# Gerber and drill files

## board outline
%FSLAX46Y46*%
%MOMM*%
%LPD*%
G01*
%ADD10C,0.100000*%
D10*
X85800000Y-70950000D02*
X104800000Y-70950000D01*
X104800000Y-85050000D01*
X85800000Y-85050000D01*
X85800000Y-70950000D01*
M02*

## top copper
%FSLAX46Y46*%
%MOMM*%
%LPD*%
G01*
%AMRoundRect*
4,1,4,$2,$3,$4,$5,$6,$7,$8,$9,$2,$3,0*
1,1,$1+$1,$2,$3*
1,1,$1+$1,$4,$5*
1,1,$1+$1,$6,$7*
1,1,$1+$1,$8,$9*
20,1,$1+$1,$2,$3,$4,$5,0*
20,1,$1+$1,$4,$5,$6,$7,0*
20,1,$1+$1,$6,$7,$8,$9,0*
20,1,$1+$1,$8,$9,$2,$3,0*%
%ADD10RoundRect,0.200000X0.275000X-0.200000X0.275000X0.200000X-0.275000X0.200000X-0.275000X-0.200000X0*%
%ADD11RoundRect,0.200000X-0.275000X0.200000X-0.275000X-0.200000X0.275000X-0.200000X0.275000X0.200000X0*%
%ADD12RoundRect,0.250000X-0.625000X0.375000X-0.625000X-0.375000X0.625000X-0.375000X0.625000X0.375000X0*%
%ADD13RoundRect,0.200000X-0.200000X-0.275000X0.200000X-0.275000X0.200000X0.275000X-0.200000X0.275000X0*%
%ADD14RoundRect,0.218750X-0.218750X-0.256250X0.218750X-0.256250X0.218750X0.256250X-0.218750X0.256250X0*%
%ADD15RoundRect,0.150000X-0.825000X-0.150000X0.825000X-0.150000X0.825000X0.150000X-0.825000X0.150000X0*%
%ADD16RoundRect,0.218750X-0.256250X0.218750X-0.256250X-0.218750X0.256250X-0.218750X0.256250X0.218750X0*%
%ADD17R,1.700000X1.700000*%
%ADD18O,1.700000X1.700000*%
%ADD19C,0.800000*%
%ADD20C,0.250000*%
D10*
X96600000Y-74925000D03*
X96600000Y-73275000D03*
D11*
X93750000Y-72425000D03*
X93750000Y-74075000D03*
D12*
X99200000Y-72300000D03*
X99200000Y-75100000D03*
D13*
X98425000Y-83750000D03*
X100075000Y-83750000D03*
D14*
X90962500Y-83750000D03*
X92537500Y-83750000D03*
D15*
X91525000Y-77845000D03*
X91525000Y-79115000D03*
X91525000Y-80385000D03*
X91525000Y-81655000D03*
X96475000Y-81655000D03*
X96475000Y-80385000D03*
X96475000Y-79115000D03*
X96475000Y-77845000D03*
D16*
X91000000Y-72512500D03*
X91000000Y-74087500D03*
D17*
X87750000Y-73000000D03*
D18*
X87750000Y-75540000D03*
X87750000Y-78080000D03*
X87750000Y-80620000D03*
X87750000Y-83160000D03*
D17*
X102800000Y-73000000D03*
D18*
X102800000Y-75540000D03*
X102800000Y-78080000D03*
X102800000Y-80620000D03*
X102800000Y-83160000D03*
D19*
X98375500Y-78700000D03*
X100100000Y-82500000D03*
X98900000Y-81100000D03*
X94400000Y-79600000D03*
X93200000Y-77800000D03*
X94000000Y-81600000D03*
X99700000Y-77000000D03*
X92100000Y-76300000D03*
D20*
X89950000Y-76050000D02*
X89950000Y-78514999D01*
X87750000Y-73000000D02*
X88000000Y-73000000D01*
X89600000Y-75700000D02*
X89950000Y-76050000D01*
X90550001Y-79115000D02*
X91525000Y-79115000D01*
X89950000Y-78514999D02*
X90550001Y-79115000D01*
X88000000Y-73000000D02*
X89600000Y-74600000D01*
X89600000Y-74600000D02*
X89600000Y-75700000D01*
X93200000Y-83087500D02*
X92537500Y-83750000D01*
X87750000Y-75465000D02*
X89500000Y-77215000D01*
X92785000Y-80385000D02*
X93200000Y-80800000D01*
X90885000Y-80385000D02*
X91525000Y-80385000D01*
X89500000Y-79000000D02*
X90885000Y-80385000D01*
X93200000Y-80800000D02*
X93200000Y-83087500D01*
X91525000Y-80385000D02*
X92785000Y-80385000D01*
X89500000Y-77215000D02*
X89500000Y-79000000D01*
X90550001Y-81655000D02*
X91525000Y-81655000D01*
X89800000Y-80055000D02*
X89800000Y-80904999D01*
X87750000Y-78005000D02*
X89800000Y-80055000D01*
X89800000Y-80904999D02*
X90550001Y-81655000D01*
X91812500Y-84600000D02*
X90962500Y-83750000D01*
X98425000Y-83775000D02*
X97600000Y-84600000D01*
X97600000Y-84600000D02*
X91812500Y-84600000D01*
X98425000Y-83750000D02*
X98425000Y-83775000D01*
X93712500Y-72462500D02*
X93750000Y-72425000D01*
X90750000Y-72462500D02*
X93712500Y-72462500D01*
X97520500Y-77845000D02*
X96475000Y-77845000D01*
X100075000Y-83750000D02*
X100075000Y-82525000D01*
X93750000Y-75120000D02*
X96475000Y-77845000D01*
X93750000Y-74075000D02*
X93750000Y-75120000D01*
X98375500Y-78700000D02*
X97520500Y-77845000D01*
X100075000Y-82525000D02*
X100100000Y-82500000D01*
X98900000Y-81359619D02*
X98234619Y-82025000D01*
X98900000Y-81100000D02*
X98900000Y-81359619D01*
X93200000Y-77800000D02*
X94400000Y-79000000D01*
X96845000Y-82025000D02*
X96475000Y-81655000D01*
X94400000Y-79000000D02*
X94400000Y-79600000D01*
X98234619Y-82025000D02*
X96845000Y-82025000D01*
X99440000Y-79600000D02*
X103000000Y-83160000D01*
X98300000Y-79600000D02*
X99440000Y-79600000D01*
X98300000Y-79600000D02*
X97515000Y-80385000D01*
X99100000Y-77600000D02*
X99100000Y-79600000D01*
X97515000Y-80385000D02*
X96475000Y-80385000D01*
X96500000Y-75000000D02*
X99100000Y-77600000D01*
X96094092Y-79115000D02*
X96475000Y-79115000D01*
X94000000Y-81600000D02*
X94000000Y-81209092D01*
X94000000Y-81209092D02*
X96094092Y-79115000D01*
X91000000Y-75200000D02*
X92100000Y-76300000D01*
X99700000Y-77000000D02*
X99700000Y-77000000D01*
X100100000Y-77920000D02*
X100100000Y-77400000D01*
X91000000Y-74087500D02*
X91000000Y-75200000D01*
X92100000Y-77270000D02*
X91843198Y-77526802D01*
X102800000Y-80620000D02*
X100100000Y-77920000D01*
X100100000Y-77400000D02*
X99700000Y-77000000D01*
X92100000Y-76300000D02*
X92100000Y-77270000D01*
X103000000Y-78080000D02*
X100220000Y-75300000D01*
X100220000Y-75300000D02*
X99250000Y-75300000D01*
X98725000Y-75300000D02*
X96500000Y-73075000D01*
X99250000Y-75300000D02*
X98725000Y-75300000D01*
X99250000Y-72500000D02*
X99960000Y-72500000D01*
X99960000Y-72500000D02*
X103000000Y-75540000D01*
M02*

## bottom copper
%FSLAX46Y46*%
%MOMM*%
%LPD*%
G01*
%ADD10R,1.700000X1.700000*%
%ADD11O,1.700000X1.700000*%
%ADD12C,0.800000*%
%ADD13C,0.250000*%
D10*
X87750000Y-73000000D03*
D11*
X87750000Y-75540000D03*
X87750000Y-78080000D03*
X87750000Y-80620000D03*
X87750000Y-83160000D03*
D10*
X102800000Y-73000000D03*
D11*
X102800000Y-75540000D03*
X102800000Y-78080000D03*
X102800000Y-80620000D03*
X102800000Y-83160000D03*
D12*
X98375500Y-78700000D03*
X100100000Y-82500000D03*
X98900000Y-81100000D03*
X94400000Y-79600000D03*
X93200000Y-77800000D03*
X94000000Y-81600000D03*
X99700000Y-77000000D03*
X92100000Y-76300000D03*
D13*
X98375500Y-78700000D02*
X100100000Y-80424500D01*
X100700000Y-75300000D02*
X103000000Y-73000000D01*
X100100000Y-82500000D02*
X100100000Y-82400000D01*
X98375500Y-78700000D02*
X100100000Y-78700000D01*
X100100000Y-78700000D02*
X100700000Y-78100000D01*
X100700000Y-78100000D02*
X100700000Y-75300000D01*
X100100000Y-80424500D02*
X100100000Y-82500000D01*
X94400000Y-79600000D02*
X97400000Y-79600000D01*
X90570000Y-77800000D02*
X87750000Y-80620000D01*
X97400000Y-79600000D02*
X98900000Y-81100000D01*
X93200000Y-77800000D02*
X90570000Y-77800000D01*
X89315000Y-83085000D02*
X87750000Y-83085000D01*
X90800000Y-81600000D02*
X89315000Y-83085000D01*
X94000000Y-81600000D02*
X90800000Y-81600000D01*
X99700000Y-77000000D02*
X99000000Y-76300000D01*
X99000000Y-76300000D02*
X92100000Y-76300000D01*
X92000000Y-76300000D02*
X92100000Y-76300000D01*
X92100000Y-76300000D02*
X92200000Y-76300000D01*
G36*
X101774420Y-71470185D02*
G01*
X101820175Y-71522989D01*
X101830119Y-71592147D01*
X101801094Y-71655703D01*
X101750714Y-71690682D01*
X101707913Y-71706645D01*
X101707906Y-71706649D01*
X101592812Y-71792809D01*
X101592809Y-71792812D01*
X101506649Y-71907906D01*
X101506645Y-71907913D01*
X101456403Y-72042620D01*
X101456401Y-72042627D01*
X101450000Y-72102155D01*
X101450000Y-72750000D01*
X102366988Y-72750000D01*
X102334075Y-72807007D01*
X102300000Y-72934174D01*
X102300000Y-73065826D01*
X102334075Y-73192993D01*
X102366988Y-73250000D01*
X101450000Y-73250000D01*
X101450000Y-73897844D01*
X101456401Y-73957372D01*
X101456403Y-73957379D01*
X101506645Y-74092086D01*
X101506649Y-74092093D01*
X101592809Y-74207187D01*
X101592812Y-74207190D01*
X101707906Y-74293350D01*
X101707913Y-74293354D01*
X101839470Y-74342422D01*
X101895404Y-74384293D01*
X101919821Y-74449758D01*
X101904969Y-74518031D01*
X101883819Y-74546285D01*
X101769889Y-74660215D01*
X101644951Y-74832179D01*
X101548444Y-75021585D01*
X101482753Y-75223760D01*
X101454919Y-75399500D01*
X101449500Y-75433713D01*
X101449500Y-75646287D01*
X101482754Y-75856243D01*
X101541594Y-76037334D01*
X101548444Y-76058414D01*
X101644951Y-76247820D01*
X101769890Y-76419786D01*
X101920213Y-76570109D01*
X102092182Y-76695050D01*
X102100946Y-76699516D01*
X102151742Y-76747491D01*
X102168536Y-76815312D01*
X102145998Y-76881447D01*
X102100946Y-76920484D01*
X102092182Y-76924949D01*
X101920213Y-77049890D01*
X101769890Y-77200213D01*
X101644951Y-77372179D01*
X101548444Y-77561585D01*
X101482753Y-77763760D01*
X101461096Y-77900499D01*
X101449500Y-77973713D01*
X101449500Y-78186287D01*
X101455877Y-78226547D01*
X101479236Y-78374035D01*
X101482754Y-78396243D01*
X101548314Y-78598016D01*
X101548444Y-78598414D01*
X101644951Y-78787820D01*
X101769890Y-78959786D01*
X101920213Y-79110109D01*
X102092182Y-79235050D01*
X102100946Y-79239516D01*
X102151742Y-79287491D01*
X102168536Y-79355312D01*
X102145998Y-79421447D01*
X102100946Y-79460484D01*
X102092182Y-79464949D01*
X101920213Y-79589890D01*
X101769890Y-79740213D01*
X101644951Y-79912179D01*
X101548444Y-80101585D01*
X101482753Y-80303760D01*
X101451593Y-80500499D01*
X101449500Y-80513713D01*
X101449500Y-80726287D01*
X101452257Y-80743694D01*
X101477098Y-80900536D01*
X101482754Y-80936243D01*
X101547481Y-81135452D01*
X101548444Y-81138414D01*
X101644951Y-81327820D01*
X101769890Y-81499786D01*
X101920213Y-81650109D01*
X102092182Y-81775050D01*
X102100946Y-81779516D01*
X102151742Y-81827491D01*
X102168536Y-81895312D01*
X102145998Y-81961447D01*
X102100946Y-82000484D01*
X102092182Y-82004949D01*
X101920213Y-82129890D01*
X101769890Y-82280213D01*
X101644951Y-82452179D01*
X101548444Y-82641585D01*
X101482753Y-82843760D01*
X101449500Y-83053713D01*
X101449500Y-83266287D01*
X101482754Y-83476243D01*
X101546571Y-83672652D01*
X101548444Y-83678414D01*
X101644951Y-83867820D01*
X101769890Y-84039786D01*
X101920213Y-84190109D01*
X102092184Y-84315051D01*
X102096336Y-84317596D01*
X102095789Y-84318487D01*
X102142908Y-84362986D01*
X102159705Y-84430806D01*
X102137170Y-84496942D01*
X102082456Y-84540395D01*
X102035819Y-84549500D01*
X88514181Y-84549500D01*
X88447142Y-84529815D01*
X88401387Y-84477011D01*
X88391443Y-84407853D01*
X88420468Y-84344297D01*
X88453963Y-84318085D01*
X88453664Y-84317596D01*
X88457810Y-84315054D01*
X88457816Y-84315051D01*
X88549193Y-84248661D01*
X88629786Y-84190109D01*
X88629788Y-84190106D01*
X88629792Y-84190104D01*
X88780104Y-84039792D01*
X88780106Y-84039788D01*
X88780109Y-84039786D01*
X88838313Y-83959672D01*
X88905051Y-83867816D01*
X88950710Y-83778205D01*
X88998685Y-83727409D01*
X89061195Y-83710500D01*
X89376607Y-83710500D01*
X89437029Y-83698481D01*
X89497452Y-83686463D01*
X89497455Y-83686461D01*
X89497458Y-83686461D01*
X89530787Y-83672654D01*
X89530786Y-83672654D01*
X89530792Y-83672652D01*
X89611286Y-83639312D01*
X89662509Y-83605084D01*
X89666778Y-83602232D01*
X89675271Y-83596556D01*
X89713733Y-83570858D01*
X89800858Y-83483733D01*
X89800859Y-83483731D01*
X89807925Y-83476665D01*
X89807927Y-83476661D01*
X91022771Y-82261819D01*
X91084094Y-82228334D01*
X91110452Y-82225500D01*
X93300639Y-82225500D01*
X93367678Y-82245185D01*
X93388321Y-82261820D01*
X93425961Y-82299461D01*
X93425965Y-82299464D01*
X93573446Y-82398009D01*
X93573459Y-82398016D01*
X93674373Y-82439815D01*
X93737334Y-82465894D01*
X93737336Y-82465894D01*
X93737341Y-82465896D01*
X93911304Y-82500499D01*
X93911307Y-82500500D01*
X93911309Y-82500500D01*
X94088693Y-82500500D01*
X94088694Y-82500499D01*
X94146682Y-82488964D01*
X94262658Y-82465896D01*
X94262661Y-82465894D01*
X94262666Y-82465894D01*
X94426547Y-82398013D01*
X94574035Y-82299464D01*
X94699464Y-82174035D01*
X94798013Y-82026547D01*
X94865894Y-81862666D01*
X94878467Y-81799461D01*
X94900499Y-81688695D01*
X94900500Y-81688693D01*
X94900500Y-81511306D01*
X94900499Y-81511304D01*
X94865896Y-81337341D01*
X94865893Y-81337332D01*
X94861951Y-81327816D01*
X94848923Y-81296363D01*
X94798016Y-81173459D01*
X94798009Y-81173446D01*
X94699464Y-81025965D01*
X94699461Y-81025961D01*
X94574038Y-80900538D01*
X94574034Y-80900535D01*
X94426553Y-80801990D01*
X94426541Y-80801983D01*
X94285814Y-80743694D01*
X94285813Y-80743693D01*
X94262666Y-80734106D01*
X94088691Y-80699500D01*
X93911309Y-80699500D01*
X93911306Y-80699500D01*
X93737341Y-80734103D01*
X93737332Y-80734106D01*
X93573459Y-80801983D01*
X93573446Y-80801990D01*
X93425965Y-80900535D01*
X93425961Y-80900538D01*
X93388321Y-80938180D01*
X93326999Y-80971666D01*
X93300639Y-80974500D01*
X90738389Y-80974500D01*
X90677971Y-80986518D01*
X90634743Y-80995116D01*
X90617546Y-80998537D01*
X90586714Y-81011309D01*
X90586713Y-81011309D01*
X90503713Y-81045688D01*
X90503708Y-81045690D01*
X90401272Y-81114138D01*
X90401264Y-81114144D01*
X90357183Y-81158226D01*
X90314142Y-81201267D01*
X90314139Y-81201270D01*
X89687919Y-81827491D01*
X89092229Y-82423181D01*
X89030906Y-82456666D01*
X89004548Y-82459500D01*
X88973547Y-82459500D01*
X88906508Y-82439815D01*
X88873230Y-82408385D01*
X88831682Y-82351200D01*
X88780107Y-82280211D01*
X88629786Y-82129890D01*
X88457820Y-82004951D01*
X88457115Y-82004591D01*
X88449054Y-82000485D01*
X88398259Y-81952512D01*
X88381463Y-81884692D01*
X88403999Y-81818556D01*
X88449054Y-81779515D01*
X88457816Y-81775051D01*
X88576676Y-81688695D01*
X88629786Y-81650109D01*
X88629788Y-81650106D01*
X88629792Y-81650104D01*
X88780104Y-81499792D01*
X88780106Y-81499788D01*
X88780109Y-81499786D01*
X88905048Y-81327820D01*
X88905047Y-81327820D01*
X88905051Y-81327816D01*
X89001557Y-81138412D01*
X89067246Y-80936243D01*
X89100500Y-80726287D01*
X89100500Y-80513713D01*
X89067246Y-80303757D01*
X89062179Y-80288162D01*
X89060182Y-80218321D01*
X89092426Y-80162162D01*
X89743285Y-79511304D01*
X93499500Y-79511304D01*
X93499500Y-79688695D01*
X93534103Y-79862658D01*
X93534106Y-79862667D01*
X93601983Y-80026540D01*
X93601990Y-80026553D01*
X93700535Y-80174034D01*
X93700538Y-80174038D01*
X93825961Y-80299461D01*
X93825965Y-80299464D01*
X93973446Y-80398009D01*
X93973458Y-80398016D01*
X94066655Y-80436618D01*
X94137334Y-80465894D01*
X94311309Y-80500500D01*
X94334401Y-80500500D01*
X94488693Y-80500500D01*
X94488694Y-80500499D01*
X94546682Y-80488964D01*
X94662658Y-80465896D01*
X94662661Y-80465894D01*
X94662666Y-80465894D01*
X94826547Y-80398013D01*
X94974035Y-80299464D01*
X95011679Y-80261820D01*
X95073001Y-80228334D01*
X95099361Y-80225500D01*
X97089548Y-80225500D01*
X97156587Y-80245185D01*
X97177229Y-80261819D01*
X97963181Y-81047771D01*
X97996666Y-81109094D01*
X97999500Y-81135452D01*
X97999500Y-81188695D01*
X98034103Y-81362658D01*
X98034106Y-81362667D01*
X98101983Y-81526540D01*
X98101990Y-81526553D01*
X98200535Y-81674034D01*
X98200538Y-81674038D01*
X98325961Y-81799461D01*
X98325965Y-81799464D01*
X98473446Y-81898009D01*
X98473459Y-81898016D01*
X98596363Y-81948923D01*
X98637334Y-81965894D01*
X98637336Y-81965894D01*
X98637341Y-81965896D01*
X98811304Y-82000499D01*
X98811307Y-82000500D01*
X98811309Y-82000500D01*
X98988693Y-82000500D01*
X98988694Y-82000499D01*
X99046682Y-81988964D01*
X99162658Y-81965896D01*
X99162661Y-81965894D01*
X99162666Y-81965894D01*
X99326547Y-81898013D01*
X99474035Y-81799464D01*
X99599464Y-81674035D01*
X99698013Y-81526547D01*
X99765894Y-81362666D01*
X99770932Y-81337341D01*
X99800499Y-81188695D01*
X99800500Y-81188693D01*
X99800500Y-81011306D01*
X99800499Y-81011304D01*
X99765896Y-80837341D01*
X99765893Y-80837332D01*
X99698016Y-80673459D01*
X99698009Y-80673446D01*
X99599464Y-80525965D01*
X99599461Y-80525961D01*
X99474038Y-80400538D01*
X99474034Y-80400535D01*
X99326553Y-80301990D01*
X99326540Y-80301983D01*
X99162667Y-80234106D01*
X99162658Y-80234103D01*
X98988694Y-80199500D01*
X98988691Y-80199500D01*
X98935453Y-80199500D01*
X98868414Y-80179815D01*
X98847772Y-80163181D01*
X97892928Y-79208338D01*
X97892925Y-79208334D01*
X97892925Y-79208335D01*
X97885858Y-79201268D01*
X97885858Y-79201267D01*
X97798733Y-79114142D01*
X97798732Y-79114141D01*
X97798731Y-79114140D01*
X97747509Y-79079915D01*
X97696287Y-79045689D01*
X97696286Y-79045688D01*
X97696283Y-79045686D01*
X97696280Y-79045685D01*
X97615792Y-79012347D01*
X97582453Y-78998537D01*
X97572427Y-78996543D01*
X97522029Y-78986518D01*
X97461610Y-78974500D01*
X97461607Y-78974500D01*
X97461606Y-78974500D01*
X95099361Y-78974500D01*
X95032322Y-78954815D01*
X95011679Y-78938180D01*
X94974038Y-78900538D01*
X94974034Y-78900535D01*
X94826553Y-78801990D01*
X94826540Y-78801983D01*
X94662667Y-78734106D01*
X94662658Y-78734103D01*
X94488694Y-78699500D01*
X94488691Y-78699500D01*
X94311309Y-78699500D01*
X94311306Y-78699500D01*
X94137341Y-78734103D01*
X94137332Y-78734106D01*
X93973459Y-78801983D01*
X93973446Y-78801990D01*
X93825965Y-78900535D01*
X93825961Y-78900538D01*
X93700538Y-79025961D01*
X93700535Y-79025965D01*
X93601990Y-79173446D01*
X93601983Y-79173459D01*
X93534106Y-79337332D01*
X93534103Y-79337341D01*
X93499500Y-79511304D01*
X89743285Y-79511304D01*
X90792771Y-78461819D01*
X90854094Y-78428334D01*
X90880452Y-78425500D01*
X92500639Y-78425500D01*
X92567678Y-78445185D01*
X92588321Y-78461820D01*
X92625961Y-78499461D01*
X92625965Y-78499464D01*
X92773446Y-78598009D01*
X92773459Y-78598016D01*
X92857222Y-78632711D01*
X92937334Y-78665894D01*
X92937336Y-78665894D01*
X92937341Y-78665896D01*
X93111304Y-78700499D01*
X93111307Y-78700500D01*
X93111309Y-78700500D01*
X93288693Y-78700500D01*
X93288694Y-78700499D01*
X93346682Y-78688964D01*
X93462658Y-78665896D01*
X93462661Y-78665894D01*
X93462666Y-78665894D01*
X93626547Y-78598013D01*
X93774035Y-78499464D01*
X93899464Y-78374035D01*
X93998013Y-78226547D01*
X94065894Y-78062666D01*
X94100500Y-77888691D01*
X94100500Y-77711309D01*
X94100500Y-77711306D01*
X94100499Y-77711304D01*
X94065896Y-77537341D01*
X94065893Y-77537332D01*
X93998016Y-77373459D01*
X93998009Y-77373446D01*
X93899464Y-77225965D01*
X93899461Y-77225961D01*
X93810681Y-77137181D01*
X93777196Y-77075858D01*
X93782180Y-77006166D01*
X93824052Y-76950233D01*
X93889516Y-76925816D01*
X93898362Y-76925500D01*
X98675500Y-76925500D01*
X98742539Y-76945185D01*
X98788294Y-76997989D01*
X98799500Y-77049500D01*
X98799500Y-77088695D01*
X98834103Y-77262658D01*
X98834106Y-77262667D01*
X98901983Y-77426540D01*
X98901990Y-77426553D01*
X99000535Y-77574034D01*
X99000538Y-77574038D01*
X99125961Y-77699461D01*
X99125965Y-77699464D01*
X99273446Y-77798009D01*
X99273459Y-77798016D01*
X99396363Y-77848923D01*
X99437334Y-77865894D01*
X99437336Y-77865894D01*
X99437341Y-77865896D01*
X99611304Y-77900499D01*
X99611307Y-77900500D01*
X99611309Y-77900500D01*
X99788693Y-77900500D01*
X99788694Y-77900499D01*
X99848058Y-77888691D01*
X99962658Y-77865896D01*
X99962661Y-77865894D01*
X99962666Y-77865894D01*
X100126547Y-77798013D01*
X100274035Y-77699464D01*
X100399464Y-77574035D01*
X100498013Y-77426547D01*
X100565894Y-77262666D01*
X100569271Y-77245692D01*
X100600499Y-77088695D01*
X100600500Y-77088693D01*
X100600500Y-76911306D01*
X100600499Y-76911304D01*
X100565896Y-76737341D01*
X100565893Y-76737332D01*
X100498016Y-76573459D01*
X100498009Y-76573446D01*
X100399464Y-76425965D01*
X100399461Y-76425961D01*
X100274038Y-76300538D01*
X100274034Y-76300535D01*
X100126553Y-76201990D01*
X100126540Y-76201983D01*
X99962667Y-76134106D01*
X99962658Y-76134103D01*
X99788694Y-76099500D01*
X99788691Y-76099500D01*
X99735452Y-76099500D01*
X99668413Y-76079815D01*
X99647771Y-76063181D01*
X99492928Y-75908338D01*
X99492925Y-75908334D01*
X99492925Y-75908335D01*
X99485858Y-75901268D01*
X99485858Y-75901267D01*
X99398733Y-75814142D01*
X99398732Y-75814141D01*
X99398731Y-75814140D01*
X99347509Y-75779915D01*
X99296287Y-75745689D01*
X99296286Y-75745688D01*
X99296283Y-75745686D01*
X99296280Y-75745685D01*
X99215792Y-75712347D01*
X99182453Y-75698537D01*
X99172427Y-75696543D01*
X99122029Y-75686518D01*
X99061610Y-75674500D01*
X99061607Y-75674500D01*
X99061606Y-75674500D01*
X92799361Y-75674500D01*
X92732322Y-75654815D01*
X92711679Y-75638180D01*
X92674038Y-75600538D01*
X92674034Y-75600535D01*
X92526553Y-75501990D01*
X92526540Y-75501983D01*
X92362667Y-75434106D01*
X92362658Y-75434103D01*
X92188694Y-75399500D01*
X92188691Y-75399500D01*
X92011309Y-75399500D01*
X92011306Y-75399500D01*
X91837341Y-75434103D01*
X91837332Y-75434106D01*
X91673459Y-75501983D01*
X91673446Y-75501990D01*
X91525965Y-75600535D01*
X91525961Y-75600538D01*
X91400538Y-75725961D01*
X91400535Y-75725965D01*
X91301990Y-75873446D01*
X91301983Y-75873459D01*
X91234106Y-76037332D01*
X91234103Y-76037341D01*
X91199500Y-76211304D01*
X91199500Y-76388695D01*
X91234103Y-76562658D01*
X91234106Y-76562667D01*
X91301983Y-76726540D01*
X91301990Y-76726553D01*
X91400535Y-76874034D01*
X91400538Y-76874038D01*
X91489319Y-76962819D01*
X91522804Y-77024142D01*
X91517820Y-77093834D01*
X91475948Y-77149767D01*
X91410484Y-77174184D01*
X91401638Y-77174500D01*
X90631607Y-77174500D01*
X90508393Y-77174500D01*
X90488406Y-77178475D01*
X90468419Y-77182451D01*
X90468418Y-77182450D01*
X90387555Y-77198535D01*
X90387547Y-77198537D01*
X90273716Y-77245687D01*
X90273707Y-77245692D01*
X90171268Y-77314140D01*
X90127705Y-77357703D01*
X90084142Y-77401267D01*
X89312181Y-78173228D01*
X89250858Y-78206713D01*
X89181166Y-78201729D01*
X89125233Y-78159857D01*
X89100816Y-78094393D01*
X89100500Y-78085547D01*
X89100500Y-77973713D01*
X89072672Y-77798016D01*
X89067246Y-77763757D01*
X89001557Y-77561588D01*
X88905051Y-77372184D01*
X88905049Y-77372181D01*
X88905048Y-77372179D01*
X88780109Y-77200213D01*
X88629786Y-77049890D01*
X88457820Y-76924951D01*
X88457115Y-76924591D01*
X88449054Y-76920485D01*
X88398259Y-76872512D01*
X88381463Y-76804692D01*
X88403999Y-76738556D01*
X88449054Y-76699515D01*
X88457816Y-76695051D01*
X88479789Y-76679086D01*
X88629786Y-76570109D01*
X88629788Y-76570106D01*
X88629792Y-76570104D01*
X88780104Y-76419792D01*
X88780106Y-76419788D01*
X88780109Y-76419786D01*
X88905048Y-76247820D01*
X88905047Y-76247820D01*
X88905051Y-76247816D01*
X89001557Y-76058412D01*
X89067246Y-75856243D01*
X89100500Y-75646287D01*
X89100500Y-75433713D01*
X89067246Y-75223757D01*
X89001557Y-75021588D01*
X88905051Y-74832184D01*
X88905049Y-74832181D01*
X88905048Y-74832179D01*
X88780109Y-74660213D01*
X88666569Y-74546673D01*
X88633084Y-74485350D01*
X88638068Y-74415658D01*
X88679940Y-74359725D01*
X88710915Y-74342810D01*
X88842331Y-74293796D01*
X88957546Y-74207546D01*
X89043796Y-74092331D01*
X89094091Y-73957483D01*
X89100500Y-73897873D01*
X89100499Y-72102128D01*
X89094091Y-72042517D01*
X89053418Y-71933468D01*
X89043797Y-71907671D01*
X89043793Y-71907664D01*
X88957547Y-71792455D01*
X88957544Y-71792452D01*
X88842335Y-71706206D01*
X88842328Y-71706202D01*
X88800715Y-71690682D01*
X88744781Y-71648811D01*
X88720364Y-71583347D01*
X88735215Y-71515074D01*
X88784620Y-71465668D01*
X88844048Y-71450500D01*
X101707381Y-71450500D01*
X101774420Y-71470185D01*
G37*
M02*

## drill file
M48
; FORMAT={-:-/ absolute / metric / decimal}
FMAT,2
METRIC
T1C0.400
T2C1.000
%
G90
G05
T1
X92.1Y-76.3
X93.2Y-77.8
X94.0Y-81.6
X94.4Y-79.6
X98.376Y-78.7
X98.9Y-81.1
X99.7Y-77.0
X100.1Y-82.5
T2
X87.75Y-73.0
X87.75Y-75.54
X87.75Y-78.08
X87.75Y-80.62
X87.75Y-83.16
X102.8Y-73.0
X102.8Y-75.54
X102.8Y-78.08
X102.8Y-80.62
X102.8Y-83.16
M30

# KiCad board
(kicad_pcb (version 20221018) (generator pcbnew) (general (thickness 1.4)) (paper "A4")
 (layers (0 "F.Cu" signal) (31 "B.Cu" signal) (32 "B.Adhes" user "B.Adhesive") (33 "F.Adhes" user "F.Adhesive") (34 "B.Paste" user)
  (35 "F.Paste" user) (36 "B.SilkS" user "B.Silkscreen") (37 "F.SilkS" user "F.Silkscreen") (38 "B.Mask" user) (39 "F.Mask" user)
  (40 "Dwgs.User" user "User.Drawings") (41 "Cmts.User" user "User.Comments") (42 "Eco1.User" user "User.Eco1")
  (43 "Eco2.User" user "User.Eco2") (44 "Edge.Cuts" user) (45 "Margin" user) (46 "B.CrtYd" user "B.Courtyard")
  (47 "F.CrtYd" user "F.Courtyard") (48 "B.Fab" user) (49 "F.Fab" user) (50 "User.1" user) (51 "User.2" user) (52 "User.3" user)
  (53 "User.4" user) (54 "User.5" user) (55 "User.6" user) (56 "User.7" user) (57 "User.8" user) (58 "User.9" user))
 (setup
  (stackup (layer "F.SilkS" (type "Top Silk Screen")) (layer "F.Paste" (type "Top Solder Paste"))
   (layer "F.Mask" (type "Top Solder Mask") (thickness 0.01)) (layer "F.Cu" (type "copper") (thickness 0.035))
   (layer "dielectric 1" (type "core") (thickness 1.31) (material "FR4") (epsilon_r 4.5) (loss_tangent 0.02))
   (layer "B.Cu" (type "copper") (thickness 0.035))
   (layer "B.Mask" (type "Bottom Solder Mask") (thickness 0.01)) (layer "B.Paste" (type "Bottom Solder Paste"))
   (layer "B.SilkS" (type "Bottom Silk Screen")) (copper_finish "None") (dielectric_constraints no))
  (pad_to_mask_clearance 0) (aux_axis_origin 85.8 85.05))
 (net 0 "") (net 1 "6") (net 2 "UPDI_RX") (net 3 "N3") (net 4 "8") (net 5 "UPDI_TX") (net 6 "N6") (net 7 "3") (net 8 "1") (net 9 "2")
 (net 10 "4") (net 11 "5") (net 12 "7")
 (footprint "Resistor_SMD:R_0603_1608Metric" (layer "F.Cu") (at 96.6 74.1 90)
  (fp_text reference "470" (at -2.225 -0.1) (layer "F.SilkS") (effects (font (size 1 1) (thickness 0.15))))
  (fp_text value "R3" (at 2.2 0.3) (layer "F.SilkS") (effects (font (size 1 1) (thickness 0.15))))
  (pad "1" smd roundrect (at -0.825 0 90) (size 0.8 0.95) (layers "F.Cu" "F.Paste" "F.Mask") (roundrect_rratio 0.25) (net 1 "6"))
  (pad "2" smd roundrect (at 0.825 0 90) (size 0.8 0.95) (layers "F.Cu" "F.Paste" "F.Mask") (roundrect_rratio 0.25) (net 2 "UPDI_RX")))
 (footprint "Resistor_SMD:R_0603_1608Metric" (layer "F.Cu") (at 93.75 73.25 -90)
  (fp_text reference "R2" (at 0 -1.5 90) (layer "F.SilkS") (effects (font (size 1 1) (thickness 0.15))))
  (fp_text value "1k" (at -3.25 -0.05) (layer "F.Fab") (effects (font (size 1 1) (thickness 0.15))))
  (pad "1" smd roundrect (at -0.825 0 270) (size 0.8 0.95) (layers "F.Cu" "F.Paste" "F.Mask") (roundrect_rratio 0.25) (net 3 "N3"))
  (pad "2" smd roundrect (at 0.825 0 270) (size 0.8 0.95) (layers "F.Cu" "F.Paste" "F.Mask") (roundrect_rratio 0.25) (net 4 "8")))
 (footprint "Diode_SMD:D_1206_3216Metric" (layer "F.Cu") (at 99.2 73.7 -90)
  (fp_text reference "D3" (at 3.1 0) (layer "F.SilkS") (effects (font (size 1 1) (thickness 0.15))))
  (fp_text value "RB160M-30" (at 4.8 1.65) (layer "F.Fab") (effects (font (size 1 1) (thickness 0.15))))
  (pad "1" smd roundrect (at -1.4 0 270) (size 1.25 1.75) (layers "F.Cu" "F.Paste" "F.Mask") (roundrect_rratio 0.2) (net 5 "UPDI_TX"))
  (pad "2" smd roundrect (at 1.4 0 270) (size 1.25 1.75) (layers "F.Cu" "F.Paste" "F.Mask") (roundrect_rratio 0.2) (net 2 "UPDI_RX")))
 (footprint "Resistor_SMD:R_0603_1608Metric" (layer "F.Cu") (at 99.25 83.75)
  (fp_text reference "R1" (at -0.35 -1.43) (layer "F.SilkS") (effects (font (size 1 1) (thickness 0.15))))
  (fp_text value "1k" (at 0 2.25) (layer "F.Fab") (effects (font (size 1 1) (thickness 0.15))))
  (pad "1" smd roundrect (at -0.825 0) (size 0.8 0.95) (layers "F.Cu" "F.Paste" "F.Mask") (roundrect_rratio 0.25) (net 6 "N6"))
  (pad "2" smd roundrect (at 0.825 0) (size 0.8 0.95) (layers "F.Cu" "F.Paste" "F.Mask") (roundrect_rratio 0.25) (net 4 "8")))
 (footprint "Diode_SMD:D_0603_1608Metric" (layer "F.Cu") (at 91.75 83.75)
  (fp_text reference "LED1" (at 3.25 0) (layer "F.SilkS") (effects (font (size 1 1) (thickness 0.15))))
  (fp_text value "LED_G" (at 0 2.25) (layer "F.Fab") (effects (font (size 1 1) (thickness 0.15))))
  (pad "1" smd roundrect (at -0.7875 0) (size 0.875 0.95) (layers "F.Cu" "F.Paste" "F.Mask") (roundrect_rratio 0.25) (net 6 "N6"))
  (pad "2" smd roundrect (at 0.7875 0) (size 0.875 0.95) (layers "F.Cu" "F.Paste" "F.Mask") (roundrect_rratio 0.25) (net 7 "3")))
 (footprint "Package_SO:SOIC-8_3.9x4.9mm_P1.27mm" (layer "F.Cu") (at 94 79.75)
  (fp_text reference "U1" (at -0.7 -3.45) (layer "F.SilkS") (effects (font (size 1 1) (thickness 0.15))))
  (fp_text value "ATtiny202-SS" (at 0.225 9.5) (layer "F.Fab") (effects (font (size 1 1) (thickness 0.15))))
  (pad "1" smd roundrect (at -2.475 -1.905) (size 1.95 0.6) (layers "F.Cu" "F.Paste" "F.Mask") (roundrect_rratio 0.25) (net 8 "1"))
  (pad "2" smd roundrect (at -2.475 -0.635) (size 1.95 0.6) (layers "F.Cu" "F.Paste" "F.Mask") (roundrect_rratio 0.25) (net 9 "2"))
  (pad "3" smd roundrect (at -2.475 0.635) (size 1.95 0.6) (layers "F.Cu" "F.Paste" "F.Mask") (roundrect_rratio 0.25) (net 7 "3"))
  (pad "4" smd roundrect (at -2.475 1.905) (size 1.95 0.6) (layers "F.Cu" "F.Paste" "F.Mask") (roundrect_rratio 0.25) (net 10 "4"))
  (pad "5" smd roundrect (at 2.475 1.905) (size 1.95 0.6) (layers "F.Cu" "F.Paste" "F.Mask") (roundrect_rratio 0.25) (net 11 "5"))
  (pad "6" smd roundrect (at 2.475 0.635) (size 1.95 0.6) (layers "F.Cu" "F.Paste" "F.Mask") (roundrect_rratio 0.25) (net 1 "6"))
  (pad "7" smd roundrect (at 2.475 -0.635) (size 1.95 0.6) (layers "F.Cu" "F.Paste" "F.Mask") (roundrect_rratio 0.25) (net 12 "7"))
  (pad "8" smd roundrect (at 2.475 -1.905) (size 1.95 0.6) (layers "F.Cu" "F.Paste" "F.Mask") (roundrect_rratio 0.25) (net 4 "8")))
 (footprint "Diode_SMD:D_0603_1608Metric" (layer "F.Cu") (at 91 73.3 -90)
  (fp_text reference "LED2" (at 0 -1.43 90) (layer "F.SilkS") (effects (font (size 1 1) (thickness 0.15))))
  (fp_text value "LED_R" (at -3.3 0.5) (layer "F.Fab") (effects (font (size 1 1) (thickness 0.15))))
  (pad "1" smd roundrect (at -0.7875 0 270) (size 0.875 0.95) (layers "F.Cu" "F.Paste" "F.Mask") (roundrect_rratio 0.25) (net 3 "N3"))
  (pad "2" smd roundrect (at 0.7875 0 270) (size 0.875 0.95) (layers "F.Cu" "F.Paste" "F.Mask") (roundrect_rratio 0.25) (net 8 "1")))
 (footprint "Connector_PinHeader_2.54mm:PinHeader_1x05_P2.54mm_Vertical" (layer "B.Cu") (at 87.75 73 180)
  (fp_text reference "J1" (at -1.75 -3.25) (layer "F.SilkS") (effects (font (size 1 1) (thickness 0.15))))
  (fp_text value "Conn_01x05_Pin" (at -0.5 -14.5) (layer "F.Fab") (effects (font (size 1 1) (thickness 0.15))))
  (pad "1" thru_hole rect (at 0 0 180) (size 1.7 1.7) (drill 1) (layers "*.Cu" "*.Mask") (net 9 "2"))
  (pad "2" thru_hole oval (at 0 -2.54 180) (size 1.7 1.7) (drill 1) (layers "*.Cu" "*.Mask") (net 7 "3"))
  (pad "3" thru_hole oval (at 0 -5.08 180) (size 1.7 1.7) (drill 1) (layers "*.Cu" "*.Mask") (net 10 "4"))
  (pad "4" thru_hole oval (at 0 -7.62 180) (size 1.7 1.7) (drill 1) (layers "*.Cu" "*.Mask") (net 11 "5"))
  (pad "5" thru_hole oval (at 0 -10.16 180) (size 1.7 1.7) (drill 1) (layers "*.Cu" "*.Mask") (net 12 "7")))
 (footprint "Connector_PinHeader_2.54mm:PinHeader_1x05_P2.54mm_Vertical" (layer "B.Cu") (at 102.8 73 180)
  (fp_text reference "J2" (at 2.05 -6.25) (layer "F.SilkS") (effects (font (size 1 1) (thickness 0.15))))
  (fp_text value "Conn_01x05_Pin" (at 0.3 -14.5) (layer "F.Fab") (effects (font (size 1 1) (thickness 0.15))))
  (pad "1" thru_hole rect (at 0 0 180) (size 1.7 1.7) (drill 1) (layers "*.Cu" "*.Mask") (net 4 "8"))
  (pad "2" thru_hole oval (at 0 -2.54 180) (size 1.7 1.7) (drill 1) (layers "*.Cu" "*.Mask") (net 5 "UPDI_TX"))
  (pad "3" thru_hole oval (at 0 -5.08 180) (size 1.7 1.7) (drill 1) (layers "*.Cu" "*.Mask") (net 2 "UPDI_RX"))
  (pad "4" thru_hole oval (at 0 -7.62 180) (size 1.7 1.7) (drill 1) (layers "*.Cu" "*.Mask") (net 8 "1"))
  (pad "5" thru_hole oval (at 0 -10.16 180) (size 1.7 1.7) (drill 1) (layers "*.Cu" "*.Mask") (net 1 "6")))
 (gr_rect (start 85.8 70.95) (end 104.8 85.05) (stroke (width 0.1) (type default)) (fill none) (layer "Edge.Cuts"))
 (segment (start 89.95 76.05) (end 89.95 78.514999) (width 0.25) (layer "F.Cu") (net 9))
 (segment (start 87.75 73) (end 88 73) (width 0.25) (layer "F.Cu") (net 9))
 (segment (start 89.6 75.7) (end 89.95 76.05) (width 0.25) (layer "F.Cu") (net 9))
 (segment (start 90.550001 79.115) (end 91.525 79.115) (width 0.25) (layer "F.Cu") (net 9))
 (segment (start 89.95 78.514999) (end 90.550001 79.115) (width 0.25) (layer "F.Cu") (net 9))
 (segment (start 88 73) (end 89.6 74.6) (width 0.25) (layer "F.Cu") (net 9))
 (segment (start 89.6 74.6) (end 89.6 75.7) (width 0.25) (layer "F.Cu") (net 9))
 (segment (start 93.2 83.0875) (end 92.5375 83.75) (width 0.25) (layer "F.Cu") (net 7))
 (segment (start 87.75 75.465) (end 89.5 77.215) (width 0.25) (layer "F.Cu") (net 7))
 (segment (start 92.785 80.385) (end 93.2 80.8) (width 0.25) (layer "F.Cu") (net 7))
 (segment (start 90.885 80.385) (end 91.525 80.385) (width 0.25) (layer "F.Cu") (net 7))
 (segment (start 89.5 79) (end 90.885 80.385) (width 0.25) (layer "F.Cu") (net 7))
 (segment (start 93.2 80.8) (end 93.2 83.0875) (width 0.25) (layer "F.Cu") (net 7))
 (segment (start 91.525 80.385) (end 92.785 80.385) (width 0.25) (layer "F.Cu") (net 7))
 (segment (start 89.5 77.215) (end 89.5 79) (width 0.25) (layer "F.Cu") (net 7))
 (segment (start 90.550001 81.655) (end 91.525 81.655) (width 0.25) (layer "F.Cu") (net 10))
 (segment (start 89.8 80.055) (end 89.8 80.904999) (width 0.25) (layer "F.Cu") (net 10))
 (segment (start 87.75 78.005) (end 89.8 80.055) (width 0.25) (layer "F.Cu") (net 10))
 (segment (start 89.8 80.904999) (end 90.550001 81.655) (width 0.25) (layer "F.Cu") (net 10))
 (segment (start 91.8125 84.6) (end 90.9625 83.75) (width 0.25) (layer "F.Cu") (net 6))
 (segment (start 98.425 83.775) (end 97.6 84.6) (width 0.25) (layer "F.Cu") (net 6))
 (segment (start 97.6 84.6) (end 91.8125 84.6) (width 0.25) (layer "F.Cu") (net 6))
 (segment (start 98.425 83.75) (end 98.425 83.775) (width 0.25) (layer "F.Cu") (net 6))
 (segment (start 93.7125 72.4625) (end 93.75 72.425) (width 0.25) (layer "F.Cu") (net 3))
 (segment (start 90.75 72.4625) (end 93.7125 72.4625) (width 0.25) (layer "F.Cu") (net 3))
 (segment (start 97.5205 77.845) (end 96.475 77.845) (width 0.25) (layer "F.Cu") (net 4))
 (segment (start 100.075 83.75) (end 100.075 82.525) (width 0.25) (layer "F.Cu") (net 4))
 (segment (start 93.75 75.12) (end 96.475 77.845) (width 0.25) (layer "F.Cu") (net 4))
 (segment (start 93.75 74.075) (end 93.75 75.12) (width 0.25) (layer "F.Cu") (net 4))
 (segment (start 98.3755 78.7) (end 97.5205 77.845) (width 0.25) (layer "F.Cu") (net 4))
 (segment (start 100.075 82.525) (end 100.1 82.5) (width 0.25) (layer "F.Cu") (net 4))
 (via (at 98.3755 78.7) (size 0.8) (drill 0.4) (layers "F.Cu" "B.Cu") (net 4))
 (via (at 100.1 82.5) (size 0.8) (drill 0.4) (layers "F.Cu" "B.Cu") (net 4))
 (segment (start 98.3755 78.7) (end 100.1 80.4245) (width 0.25) (layer "B.Cu") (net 4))
 (segment (start 100.7 75.3) (end 103 73) (width 0.25) (layer "B.Cu") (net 4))
 (segment (start 100.1 82.5) (end 100.1 82.4) (width 0.25) (layer "B.Cu") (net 4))
 (segment (start 98.3755 78.7) (end 100.1 78.7) (width 0.25) (layer "B.Cu") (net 4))
 (segment (start 100.1 78.7) (end 100.7 78.1) (width 0.25) (layer "B.Cu") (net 4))
 (segment (start 100.7 78.1) (end 100.7 75.3) (width 0.25) (layer "B.Cu") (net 4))
 (segment (start 100.1 80.4245) (end 100.1 82.5) (width 0.25) (layer "B.Cu") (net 4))
 (segment (start 98.9 81.359619) (end 98.234619 82.025) (width 0.25) (layer "F.Cu") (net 11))
 (segment (start 98.9 81.1) (end 98.9 81.359619) (width 0.25) (layer "F.Cu") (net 11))
 (segment (start 93.2 77.8) (end 94.4 79) (width 0.25) (layer "F.Cu") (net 11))
 (segment (start 96.845 82.025) (end 96.475 81.655) (width 0.25) (layer "F.Cu") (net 11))
 (segment (start 94.4 79) (end 94.4 79.6) (width 0.25) (layer "F.Cu") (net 11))
 (segment (start 98.234619 82.025) (end 96.845 82.025) (width 0.25) (layer "F.Cu") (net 11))
 (via (at 98.9 81.1) (size 0.8) (drill 0.4) (layers "F.Cu" "B.Cu") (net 11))
 (via (at 94.4 79.6) (size 0.8) (drill 0.4) (layers "F.Cu" "B.Cu") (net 11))
 (via (at 93.2 77.8) (size 0.8) (drill 0.4) (layers "F.Cu" "B.Cu") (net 11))
 (segment (start 94.4 79.6) (end 97.4 79.6) (width 0.25) (layer "B.Cu") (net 11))
 (segment (start 90.57 77.8) (end 87.75 80.62) (width 0.25) (layer "B.Cu") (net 11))
 (segment (start 97.4 79.6) (end 98.9 81.1) (width 0.25) (layer "B.Cu") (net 11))
 (segment (start 93.2 77.8) (end 90.57 77.8) (width 0.25) (layer "B.Cu") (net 11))
 (segment (start 99.44 79.6) (end 103 83.16) (width 0.25) (layer "F.Cu") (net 1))
 (segment (start 98.3 79.6) (end 99.44 79.6) (width 0.25) (layer "F.Cu") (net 1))
 (segment (start 98.3 79.6) (end 97.515 80.385) (width 0.25) (layer "F.Cu") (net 1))
 (segment (start 99.1 77.6) (end 99.1 79.6) (width 0.25) (layer "F.Cu") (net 1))
 (segment (start 97.515 80.385) (end 96.475 80.385) (width 0.25) (layer "F.Cu") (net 1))
 (segment (start 96.5 75) (end 99.1 77.6) (width 0.25) (layer "F.Cu") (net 1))
 (segment (start 96.094092 79.115) (end 96.475 79.115) (width 0.25) (layer "F.Cu") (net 12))
 (segment (start 94 81.6) (end 94 81.209092) (width 0.25) (layer "F.Cu") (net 12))
 (segment (start 94 81.209092) (end 96.094092 79.115) (width 0.25) (layer "F.Cu") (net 12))
 (via (at 94 81.6) (size 0.8) (drill 0.4) (layers "F.Cu" "B.Cu") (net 12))
 (segment (start 89.315 83.085) (end 87.75 83.085) (width 0.25) (layer "B.Cu") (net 12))
 (segment (start 90.8 81.6) (end 89.315 83.085) (width 0.25) (layer "B.Cu") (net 12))
 (segment (start 94 81.6) (end 90.8 81.6) (width 0.25) (layer "B.Cu") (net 12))
 (segment (start 91 75.2) (end 92.1 76.3) (width 0.25) (layer "F.Cu") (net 8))
 (segment (start 99.7 77) (end 99.7 77) (width 0.25) (layer "F.Cu") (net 8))
 (segment (start 100.1 77.92) (end 100.1 77.4) (width 0.25) (layer "F.Cu") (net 8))
 (segment (start 91 74.0875) (end 91 75.2) (width 0.25) (layer "F.Cu") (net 8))
 (segment (start 92.1 77.27) (end 91.843198 77.526802) (width 0.25) (layer "F.Cu") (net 8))
 (segment (start 102.8 80.62) (end 100.1 77.92) (width 0.25) (layer "F.Cu") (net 8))
 (segment (start 100.1 77.4) (end 99.7 77) (width 0.25) (layer "F.Cu") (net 8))
 (segment (start 92.1 76.3) (end 92.1 77.27) (width 0.25) (layer "F.Cu") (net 8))
 (via (at 99.7 77) (size 0.8) (drill 0.4) (layers "F.Cu" "B.Cu") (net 8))
 (via (at 92.1 76.3) (size 0.8) (drill 0.4) (layers "F.Cu" "B.Cu") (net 8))
 (segment (start 99.7 77) (end 99 76.3) (width 0.25) (layer "B.Cu") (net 8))
 (segment (start 99 76.3) (end 92.1 76.3) (width 0.25) (layer "B.Cu") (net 8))
 (segment (start 92 76.3) (end 92.1 76.3) (width 0.25) (layer "B.Cu") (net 8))
 (segment (start 92.1 76.3) (end 92.2 76.3) (width 0.25) (layer "B.Cu") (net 8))
 (segment (start 103 78.08) (end 100.22 75.3) (width 0.25) (layer "F.Cu") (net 2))
 (segment (start 100.22 75.3) (end 99.25 75.3) (width 0.25) (layer "F.Cu") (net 2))
 (segment (start 98.725 75.3) (end 96.5 73.075) (width 0.25) (layer "F.Cu") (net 2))
 (segment (start 99.25 75.3) (end 98.725 75.3) (width 0.25) (layer "F.Cu") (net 2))
 (segment (start 99.25 72.5) (end 99.96 72.5) (width 0.25) (layer "F.Cu") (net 5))
 (segment (start 99.96 72.5) (end 103 75.54) (width 0.25) (layer "F.Cu") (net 5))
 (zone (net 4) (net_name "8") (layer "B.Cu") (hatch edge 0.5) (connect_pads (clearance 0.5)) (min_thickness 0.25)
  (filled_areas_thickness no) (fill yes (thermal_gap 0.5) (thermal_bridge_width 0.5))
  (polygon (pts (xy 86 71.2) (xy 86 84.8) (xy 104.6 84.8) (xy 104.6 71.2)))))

